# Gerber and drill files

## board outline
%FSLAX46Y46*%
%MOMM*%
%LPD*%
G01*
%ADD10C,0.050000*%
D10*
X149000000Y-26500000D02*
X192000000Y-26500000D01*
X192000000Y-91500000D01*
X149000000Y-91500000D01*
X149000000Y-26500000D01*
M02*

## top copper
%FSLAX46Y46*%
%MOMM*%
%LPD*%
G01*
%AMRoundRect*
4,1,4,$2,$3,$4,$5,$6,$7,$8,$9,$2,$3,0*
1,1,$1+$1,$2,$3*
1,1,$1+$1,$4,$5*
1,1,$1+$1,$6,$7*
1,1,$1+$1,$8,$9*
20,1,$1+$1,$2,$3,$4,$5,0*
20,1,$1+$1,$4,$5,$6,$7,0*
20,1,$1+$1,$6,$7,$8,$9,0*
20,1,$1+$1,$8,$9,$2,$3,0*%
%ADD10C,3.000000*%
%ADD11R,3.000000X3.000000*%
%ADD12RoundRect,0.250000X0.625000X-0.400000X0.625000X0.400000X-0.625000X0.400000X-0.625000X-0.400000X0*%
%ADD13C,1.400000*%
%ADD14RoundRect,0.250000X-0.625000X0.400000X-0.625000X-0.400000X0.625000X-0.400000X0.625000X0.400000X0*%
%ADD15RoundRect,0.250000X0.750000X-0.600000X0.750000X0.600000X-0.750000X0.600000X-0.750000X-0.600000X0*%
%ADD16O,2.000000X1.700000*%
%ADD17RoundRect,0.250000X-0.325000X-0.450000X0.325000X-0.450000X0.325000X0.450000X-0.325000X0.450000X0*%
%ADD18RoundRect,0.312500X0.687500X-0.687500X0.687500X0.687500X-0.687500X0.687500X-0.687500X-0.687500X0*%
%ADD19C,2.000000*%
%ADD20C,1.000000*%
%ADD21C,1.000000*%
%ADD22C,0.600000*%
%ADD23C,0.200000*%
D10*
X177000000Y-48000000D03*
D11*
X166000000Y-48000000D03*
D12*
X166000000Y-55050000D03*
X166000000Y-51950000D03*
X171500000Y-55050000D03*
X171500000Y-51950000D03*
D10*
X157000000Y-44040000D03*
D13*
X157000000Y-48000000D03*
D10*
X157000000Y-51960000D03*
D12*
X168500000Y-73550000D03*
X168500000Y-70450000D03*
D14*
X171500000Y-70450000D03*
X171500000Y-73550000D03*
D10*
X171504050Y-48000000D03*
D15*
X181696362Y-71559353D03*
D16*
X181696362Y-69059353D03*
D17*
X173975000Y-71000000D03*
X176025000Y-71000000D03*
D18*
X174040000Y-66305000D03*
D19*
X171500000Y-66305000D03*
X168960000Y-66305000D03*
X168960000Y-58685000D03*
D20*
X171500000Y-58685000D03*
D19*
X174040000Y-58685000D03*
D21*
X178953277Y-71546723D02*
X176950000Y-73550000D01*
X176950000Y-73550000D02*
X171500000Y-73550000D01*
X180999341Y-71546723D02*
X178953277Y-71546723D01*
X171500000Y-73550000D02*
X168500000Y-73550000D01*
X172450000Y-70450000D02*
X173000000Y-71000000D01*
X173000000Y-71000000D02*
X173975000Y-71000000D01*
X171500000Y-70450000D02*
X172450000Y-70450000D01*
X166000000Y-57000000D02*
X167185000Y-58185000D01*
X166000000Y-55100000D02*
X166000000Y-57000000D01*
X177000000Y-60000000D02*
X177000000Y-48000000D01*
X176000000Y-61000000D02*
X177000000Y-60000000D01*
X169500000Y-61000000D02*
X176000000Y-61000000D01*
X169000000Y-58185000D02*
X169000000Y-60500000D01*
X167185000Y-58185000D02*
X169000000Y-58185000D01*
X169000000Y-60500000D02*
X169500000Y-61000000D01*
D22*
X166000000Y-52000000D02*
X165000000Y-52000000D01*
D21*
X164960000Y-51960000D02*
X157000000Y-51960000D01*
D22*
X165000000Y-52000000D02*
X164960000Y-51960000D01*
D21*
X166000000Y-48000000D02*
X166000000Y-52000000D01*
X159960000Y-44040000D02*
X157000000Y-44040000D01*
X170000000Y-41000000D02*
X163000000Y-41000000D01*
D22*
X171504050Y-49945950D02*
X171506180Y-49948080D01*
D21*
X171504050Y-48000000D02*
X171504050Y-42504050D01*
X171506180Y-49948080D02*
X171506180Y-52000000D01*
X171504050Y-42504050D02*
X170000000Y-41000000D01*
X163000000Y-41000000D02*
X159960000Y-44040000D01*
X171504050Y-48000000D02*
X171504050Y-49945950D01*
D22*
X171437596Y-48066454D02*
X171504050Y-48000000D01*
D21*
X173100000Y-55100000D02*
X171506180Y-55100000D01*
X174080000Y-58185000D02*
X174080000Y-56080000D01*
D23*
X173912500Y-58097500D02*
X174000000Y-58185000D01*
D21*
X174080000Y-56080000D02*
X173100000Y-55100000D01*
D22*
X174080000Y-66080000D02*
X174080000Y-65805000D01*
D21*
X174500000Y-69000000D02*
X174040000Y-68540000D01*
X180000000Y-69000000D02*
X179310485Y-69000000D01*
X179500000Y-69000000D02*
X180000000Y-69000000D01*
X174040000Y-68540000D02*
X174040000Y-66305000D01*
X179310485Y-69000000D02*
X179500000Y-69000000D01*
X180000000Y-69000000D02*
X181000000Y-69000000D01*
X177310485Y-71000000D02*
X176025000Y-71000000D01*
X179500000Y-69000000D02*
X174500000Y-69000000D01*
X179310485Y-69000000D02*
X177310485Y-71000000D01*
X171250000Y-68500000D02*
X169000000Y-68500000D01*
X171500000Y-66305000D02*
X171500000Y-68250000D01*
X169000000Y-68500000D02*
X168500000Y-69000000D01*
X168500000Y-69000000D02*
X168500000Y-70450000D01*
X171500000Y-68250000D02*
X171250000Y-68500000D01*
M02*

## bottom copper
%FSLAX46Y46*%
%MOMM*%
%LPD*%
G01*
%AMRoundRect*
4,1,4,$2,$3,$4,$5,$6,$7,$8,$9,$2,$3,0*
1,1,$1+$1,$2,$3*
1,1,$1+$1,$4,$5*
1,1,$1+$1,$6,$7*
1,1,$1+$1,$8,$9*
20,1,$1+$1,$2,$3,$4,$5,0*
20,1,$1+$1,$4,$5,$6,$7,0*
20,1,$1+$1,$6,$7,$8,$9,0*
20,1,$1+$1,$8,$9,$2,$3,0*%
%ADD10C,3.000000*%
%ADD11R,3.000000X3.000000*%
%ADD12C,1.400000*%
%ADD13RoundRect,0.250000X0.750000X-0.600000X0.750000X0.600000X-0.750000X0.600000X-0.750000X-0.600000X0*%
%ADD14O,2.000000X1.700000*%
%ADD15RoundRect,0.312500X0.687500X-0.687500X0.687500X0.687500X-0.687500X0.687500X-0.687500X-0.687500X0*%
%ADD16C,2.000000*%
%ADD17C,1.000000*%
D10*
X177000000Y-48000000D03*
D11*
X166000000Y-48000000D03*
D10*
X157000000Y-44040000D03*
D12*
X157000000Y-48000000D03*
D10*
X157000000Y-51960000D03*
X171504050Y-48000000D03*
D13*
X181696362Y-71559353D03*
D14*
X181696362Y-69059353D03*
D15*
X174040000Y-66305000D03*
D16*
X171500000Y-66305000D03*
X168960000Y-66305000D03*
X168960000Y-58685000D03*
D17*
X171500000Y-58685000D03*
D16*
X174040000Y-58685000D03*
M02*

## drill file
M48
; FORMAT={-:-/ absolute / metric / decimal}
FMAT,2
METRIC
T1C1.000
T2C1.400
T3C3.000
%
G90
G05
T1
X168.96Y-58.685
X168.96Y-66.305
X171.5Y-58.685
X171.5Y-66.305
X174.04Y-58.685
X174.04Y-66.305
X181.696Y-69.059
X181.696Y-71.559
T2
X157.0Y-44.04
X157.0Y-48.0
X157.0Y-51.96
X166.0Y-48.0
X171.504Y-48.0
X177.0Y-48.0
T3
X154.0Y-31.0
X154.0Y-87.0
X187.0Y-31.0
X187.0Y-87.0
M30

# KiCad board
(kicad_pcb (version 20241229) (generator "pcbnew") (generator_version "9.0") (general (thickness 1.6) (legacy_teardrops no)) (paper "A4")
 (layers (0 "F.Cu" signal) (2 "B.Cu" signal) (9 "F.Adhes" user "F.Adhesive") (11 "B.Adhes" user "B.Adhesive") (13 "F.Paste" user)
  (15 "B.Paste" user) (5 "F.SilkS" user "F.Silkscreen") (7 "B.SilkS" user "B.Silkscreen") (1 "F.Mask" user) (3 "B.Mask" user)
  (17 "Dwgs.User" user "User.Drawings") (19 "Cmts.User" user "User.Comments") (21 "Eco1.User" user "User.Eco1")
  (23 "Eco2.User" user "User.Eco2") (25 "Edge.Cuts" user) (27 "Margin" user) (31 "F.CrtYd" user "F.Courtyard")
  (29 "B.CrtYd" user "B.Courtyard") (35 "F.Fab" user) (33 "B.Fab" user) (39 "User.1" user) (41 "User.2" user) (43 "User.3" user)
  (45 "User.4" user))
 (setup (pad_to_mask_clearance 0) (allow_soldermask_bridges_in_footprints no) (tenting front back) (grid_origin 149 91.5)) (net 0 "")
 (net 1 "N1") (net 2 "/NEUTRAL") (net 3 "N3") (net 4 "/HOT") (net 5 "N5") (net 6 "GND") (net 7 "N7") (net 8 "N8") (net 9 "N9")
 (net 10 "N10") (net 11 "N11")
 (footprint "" (layer "F.Cu") (at 177 48)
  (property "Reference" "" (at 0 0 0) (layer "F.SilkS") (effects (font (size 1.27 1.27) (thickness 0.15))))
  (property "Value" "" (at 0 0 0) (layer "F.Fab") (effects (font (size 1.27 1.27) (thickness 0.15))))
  (pad "3" thru_hole circle (at 0 0) (size 3 3) (drill 1.4) (layers "*.Cu" "*.Mask") (remove_unused_layers no) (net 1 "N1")))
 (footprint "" (layer "F.Cu") (at 166 48)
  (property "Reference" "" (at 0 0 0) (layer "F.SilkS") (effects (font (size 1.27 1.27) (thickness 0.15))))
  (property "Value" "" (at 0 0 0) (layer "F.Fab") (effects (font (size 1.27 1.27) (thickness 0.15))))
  (pad "1" thru_hole rect (at 0 0) (size 3 3) (drill 1.4) (layers "*.Cu" "*.Mask") (remove_unused_layers no) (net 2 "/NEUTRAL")))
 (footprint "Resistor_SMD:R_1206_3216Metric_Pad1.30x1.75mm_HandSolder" (layer "F.Cu") (at 166 53.5 90)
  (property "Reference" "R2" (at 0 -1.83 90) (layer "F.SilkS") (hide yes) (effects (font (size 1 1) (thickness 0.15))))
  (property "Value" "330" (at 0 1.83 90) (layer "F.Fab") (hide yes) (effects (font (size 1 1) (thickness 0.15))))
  (pad "1" smd roundrect (at -1.55 0 90) (size 1.3 1.75) (layers "F.Cu" "F.Mask" "F.Paste") (roundrect_rratio 0.192308) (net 1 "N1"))
  (pad "2" smd roundrect (at 1.55 0 90) (size 1.3 1.75) (layers "F.Cu" "F.Mask" "F.Paste") (roundrect_rratio 0.192308) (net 2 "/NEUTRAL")))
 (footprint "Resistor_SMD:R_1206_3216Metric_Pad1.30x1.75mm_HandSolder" (layer "F.Cu") (at 171.5 53.5 90)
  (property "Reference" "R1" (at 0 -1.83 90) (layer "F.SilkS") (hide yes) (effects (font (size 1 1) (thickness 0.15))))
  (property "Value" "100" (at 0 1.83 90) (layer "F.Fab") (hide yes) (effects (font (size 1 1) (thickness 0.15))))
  (pad "1" smd roundrect (at -1.55 0 90) (size 1.3 1.75) (layers "F.Cu" "F.Mask" "F.Paste") (roundrect_rratio 0.192308) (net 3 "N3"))
  (pad "2" smd roundrect (at 1.55 0 90) (size 1.3 1.75) (layers "F.Cu" "F.Mask" "F.Paste") (roundrect_rratio 0.192308) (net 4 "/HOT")))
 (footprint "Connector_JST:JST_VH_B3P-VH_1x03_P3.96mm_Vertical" (layer "F.Cu") (at 157 44.04 -90)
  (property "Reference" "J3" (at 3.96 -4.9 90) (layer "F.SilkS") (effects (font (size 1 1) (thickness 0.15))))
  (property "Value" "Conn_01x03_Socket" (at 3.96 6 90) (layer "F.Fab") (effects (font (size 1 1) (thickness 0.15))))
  (pad "1" thru_hole circle (at 0 0 270) (size 3 3) (drill 1.4) (layers "*.Cu" "*.Mask") (remove_unused_layers no) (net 4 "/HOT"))
  (pad "2" thru_hole circle (at 3.96 0 270) (size 1.4 1.4) (drill 1.4) (layers "*.Cu" "*.Mask") (remove_unused_layers no) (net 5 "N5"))
  (pad "3" thru_hole circle (at 7.92 0 270) (size 3 3) (drill 1.4) (layers "*.Cu" "*.Mask") (remove_unused_layers no) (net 2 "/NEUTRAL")))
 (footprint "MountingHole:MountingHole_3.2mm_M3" (layer "F.Cu") (at 154 87)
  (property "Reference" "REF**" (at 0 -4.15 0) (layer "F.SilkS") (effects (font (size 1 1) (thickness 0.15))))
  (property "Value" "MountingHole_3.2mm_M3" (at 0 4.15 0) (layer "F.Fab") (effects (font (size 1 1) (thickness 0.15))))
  (pad "" np_thru_hole circle (at 0 0) (size 3 3) (drill 3) (layers "*.Cu" "*.Mask")))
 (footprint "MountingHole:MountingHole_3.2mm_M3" (layer "F.Cu") (at 154 31)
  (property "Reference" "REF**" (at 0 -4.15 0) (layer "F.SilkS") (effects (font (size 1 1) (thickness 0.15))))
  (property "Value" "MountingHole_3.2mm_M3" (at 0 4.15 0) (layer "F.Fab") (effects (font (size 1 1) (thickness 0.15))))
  (pad "" np_thru_hole circle (at 0 0) (size 3 3) (drill 3) (layers "*.Cu" "*.Mask")))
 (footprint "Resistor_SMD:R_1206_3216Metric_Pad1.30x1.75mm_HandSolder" (layer "F.Cu") (at 168.5 72 90)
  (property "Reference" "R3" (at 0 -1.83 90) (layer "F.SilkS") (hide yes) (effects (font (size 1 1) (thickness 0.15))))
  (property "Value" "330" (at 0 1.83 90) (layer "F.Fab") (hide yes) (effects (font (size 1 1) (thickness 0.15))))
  (pad "1" smd roundrect (at -1.55 0 90) (size 1.3 1.75) (layers "F.Cu" "F.Mask" "F.Paste") (roundrect_rratio 0.192308) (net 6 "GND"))
  (pad "2" smd roundrect (at 1.55 0 90) (size 1.3 1.75) (layers "F.Cu" "F.Mask" "F.Paste") (roundrect_rratio 0.192308) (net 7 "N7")))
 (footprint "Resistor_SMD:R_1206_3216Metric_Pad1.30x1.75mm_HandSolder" (layer "F.Cu") (at 171.5 72 -90)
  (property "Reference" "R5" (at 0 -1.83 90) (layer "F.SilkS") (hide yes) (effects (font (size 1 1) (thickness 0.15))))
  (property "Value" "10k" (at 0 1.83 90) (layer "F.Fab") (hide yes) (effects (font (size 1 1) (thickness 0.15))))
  (pad "1" smd roundrect (at -1.55 0 270) (size 1.3 1.75) (layers "F.Cu" "F.Mask" "F.Paste") (roundrect_rratio 0.192308) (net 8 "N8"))
  (pad "2" smd roundrect (at 1.55 0 270) (size 1.3 1.75) (layers "F.Cu" "F.Mask" "F.Paste") (roundrect_rratio 0.192308) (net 6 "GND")))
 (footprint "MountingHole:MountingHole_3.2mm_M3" (layer "F.Cu") (at 187 87)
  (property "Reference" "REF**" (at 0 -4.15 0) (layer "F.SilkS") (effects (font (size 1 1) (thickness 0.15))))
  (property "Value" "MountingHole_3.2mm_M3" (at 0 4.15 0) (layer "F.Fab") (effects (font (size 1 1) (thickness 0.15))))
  (pad "" np_thru_hole circle (at 0 0) (size 3 3) (drill 3) (layers "*.Cu" "*.Mask")))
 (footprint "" (layer "F.Cu") (at 171.50405 48)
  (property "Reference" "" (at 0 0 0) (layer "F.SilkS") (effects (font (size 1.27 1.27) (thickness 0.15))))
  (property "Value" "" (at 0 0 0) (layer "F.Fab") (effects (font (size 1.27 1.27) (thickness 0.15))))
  (pad "2" thru_hole circle (at 0 0) (size 3 3) (drill 1.4) (layers "*.Cu" "*.Mask") (remove_unused_layers no) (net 4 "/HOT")))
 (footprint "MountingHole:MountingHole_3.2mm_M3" (layer "F.Cu") (at 187 31)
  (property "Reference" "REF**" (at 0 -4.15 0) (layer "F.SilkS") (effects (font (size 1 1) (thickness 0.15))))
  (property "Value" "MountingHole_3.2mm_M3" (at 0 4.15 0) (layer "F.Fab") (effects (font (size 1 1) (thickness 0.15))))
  (pad "" np_thru_hole circle (at 0 0) (size 3 3) (drill 3) (layers "*.Cu" "*.Mask")))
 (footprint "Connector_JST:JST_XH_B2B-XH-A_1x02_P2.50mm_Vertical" (layer "F.Cu") (at 181.696362 71.559353 90)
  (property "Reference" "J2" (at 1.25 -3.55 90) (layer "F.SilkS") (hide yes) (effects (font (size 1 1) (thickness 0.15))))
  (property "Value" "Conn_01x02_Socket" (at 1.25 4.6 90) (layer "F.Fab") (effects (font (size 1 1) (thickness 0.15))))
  (pad "1" thru_hole roundrect (at 0 0 90) (size 1.7 2) (drill 1) (layers "*.Cu" "*.Mask") (remove_unused_layers no)
   (roundrect_rratio 0.147059) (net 6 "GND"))
  (pad "2" thru_hole oval (at 2.5 0 90) (size 1.7 2) (drill 1) (layers "*.Cu" "*.Mask") (remove_unused_layers no) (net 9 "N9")))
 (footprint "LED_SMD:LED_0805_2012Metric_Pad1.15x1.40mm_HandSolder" (layer "F.Cu") (at 175 71)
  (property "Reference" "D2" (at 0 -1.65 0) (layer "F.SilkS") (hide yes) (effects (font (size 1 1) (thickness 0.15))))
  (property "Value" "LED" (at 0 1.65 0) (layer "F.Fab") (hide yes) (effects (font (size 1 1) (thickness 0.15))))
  (pad "1" smd roundrect (at -1.025 0) (size 1.15 1.4) (layers "F.Cu" "F.Mask" "F.Paste") (roundrect_rratio 0.217391) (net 8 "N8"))
  (pad "2" smd roundrect (at 1.025 0) (size 1.15 1.4) (layers "F.Cu" "F.Mask" "F.Paste") (roundrect_rratio 0.217391) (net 9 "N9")))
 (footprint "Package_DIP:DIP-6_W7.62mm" (layer "B.Cu") (at 174.04 66.305 90)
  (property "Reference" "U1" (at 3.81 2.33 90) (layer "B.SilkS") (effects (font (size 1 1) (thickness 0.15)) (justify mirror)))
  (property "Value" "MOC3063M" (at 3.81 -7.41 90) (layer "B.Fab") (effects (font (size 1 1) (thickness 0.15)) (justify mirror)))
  (pad "1" thru_hole roundrect (at 0 0 90) (size 2 2) (drill 1) (layers "*.Cu" "*.Mask") (remove_unused_layers no)
   (roundrect_rratio 0.15625) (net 9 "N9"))
  (pad "2" thru_hole circle (at 0 -2.54 90) (size 2 2) (drill 1) (layers "*.Cu" "*.Mask") (remove_unused_layers no) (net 7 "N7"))
  (pad "3" thru_hole circle (at 0 -5.08 90) (size 2 2) (drill 1) (layers "*.Cu" "*.Mask") (remove_unused_layers no) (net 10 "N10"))
  (pad "4" thru_hole circle (at 7.62 -5.08 90) (size 2 2) (drill 1) (layers "*.Cu" "*.Mask") (remove_unused_layers no) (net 1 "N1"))
  (pad "5" thru_hole circle (at 7.62 -2.54 90) (size 1 1) (drill 1) (layers "*.Cu" "*.Mask") (remove_unused_layers no) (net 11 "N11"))
  (pad "6" thru_hole circle (at 7.62 0 90) (size 2 2) (drill 1) (layers "*.Cu" "*.Mask") (remove_unused_layers no) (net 3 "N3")))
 (gr_rect (start 149 26.5) (end 192 91.5) (stroke (width 0.05) (type default)) (fill no) (layer "Edge.Cuts"))
 (segment (start 178.953277 71.546723) (end 176.95 73.55) (width 1) (layer "F.Cu") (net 6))
 (segment (start 176.95 73.55) (end 171.5 73.55) (width 1) (layer "F.Cu") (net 6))
 (segment (start 180.999341 71.546723) (end 178.953277 71.546723) (width 1) (layer "F.Cu") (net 6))
 (segment (start 171.5 73.55) (end 168.5 73.55) (width 1) (layer "F.Cu") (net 6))
 (segment (start 172.45 70.45) (end 173 71) (width 1) (layer "F.Cu") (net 8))
 (segment (start 173 71) (end 173.975 71) (width 1) (layer "F.Cu") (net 8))
 (segment (start 171.5 70.45) (end 172.45 70.45) (width 1) (layer "F.Cu") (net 8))
 (segment (start 166 57) (end 167.185 58.185) (width 1) (layer "F.Cu") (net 1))
 (segment (start 166 55.1) (end 166 57) (width 1) (layer "F.Cu") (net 1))
 (segment (start 177 60) (end 177 48) (width 1) (layer "F.Cu") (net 1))
 (segment (start 176 61) (end 177 60) (width 1) (layer "F.Cu") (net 1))
 (segment (start 169.5 61) (end 176 61) (width 1) (layer "F.Cu") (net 1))
 (segment (start 169 58.185) (end 169 60.5) (width 1) (layer "F.Cu") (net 1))
 (segment (start 167.185 58.185) (end 169 58.185) (width 1) (layer "F.Cu") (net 1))
 (segment (start 169 60.5) (end 169.5 61) (width 1) (layer "F.Cu") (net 1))
 (segment (start 166 52) (end 165 52) (width 0.6) (layer "F.Cu") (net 2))
 (segment (start 164.96 51.96) (end 157 51.96) (width 1) (layer "F.Cu") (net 2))
 (segment (start 165 52) (end 164.96 51.96) (width 0.6) (layer "F.Cu") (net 2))
 (segment (start 166 48) (end 166 52) (width 1) (layer "F.Cu") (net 2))
 (segment (start 159.96 44.04) (end 157 44.04) (width 1) (layer "F.Cu") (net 4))
 (segment (start 170 41) (end 163 41) (width 1) (layer "F.Cu") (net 4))
 (segment (start 171.50405 49.94595) (end 171.50618 49.94808) (width 0.6) (layer "F.Cu") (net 4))
 (segment (start 171.50405 48) (end 171.50405 42.50405) (width 1) (layer "F.Cu") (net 4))
 (segment (start 171.50618 49.94808) (end 171.50618 52) (width 1) (layer "F.Cu") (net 4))
 (segment (start 171.50405 42.50405) (end 170 41) (width 1) (layer "F.Cu") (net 4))
 (segment (start 163 41) (end 159.96 44.04) (width 1) (layer "F.Cu") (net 4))
 (segment (start 171.50405 48) (end 171.50405 49.94595) (width 1) (layer "F.Cu") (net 4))
 (segment (start 171.437596 48.066454) (end 171.50405 48) (width 0.6) (layer "F.Cu") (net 4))
 (segment (start 173.1 55.1) (end 171.50618 55.1) (width 1) (layer "F.Cu") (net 3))
 (segment (start 174.08 58.185) (end 174.08 56.08) (width 1) (layer "F.Cu") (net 3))
 (segment (start 173.9125 58.0975) (end 174 58.185) (width 0.2) (layer "F.Cu") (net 3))
 (segment (start 174.08 56.08) (end 173.1 55.1) (width 1) (layer "F.Cu") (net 3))
 (segment (start 174.08 66.08) (end 174.08 65.805) (width 0.6) (layer "F.Cu") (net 9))
 (segment (start 174.5 69) (end 174.04 68.54) (width 1) (layer "F.Cu") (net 9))
 (segment (start 180 69) (end 179.310485 69) (width 1) (layer "F.Cu") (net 9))
 (segment (start 179.5 69) (end 180 69) (width 1) (layer "F.Cu") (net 9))
 (segment (start 174.04 68.54) (end 174.04 66.305) (width 1) (layer "F.Cu") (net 9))
 (segment (start 179.310485 69) (end 179.5 69) (width 1) (layer "F.Cu") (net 9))
 (segment (start 180 69) (end 181 69) (width 1) (layer "F.Cu") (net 9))
 (segment (start 177.310485 71) (end 176.025 71) (width 1) (layer "F.Cu") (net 9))
 (segment (start 179.5 69) (end 174.5 69) (width 1) (layer "F.Cu") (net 9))
 (segment (start 179.310485 69) (end 177.310485 71) (width 1) (layer "F.Cu") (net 9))
 (segment (start 171.25 68.5) (end 169 68.5) (width 1) (layer "F.Cu") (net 7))
 (segment (start 171.5 66.305) (end 171.5 68.25) (width 1) (layer "F.Cu") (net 7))
 (segment (start 169 68.5) (end 168.5 69) (width 1) (layer "F.Cu") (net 7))
 (segment (start 168.5 69) (end 168.5 70.45) (width 1) (layer "F.Cu") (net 7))
 (segment (start 171.5 68.25) (end 171.25 68.5) (width 1) (layer "F.Cu") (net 7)))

